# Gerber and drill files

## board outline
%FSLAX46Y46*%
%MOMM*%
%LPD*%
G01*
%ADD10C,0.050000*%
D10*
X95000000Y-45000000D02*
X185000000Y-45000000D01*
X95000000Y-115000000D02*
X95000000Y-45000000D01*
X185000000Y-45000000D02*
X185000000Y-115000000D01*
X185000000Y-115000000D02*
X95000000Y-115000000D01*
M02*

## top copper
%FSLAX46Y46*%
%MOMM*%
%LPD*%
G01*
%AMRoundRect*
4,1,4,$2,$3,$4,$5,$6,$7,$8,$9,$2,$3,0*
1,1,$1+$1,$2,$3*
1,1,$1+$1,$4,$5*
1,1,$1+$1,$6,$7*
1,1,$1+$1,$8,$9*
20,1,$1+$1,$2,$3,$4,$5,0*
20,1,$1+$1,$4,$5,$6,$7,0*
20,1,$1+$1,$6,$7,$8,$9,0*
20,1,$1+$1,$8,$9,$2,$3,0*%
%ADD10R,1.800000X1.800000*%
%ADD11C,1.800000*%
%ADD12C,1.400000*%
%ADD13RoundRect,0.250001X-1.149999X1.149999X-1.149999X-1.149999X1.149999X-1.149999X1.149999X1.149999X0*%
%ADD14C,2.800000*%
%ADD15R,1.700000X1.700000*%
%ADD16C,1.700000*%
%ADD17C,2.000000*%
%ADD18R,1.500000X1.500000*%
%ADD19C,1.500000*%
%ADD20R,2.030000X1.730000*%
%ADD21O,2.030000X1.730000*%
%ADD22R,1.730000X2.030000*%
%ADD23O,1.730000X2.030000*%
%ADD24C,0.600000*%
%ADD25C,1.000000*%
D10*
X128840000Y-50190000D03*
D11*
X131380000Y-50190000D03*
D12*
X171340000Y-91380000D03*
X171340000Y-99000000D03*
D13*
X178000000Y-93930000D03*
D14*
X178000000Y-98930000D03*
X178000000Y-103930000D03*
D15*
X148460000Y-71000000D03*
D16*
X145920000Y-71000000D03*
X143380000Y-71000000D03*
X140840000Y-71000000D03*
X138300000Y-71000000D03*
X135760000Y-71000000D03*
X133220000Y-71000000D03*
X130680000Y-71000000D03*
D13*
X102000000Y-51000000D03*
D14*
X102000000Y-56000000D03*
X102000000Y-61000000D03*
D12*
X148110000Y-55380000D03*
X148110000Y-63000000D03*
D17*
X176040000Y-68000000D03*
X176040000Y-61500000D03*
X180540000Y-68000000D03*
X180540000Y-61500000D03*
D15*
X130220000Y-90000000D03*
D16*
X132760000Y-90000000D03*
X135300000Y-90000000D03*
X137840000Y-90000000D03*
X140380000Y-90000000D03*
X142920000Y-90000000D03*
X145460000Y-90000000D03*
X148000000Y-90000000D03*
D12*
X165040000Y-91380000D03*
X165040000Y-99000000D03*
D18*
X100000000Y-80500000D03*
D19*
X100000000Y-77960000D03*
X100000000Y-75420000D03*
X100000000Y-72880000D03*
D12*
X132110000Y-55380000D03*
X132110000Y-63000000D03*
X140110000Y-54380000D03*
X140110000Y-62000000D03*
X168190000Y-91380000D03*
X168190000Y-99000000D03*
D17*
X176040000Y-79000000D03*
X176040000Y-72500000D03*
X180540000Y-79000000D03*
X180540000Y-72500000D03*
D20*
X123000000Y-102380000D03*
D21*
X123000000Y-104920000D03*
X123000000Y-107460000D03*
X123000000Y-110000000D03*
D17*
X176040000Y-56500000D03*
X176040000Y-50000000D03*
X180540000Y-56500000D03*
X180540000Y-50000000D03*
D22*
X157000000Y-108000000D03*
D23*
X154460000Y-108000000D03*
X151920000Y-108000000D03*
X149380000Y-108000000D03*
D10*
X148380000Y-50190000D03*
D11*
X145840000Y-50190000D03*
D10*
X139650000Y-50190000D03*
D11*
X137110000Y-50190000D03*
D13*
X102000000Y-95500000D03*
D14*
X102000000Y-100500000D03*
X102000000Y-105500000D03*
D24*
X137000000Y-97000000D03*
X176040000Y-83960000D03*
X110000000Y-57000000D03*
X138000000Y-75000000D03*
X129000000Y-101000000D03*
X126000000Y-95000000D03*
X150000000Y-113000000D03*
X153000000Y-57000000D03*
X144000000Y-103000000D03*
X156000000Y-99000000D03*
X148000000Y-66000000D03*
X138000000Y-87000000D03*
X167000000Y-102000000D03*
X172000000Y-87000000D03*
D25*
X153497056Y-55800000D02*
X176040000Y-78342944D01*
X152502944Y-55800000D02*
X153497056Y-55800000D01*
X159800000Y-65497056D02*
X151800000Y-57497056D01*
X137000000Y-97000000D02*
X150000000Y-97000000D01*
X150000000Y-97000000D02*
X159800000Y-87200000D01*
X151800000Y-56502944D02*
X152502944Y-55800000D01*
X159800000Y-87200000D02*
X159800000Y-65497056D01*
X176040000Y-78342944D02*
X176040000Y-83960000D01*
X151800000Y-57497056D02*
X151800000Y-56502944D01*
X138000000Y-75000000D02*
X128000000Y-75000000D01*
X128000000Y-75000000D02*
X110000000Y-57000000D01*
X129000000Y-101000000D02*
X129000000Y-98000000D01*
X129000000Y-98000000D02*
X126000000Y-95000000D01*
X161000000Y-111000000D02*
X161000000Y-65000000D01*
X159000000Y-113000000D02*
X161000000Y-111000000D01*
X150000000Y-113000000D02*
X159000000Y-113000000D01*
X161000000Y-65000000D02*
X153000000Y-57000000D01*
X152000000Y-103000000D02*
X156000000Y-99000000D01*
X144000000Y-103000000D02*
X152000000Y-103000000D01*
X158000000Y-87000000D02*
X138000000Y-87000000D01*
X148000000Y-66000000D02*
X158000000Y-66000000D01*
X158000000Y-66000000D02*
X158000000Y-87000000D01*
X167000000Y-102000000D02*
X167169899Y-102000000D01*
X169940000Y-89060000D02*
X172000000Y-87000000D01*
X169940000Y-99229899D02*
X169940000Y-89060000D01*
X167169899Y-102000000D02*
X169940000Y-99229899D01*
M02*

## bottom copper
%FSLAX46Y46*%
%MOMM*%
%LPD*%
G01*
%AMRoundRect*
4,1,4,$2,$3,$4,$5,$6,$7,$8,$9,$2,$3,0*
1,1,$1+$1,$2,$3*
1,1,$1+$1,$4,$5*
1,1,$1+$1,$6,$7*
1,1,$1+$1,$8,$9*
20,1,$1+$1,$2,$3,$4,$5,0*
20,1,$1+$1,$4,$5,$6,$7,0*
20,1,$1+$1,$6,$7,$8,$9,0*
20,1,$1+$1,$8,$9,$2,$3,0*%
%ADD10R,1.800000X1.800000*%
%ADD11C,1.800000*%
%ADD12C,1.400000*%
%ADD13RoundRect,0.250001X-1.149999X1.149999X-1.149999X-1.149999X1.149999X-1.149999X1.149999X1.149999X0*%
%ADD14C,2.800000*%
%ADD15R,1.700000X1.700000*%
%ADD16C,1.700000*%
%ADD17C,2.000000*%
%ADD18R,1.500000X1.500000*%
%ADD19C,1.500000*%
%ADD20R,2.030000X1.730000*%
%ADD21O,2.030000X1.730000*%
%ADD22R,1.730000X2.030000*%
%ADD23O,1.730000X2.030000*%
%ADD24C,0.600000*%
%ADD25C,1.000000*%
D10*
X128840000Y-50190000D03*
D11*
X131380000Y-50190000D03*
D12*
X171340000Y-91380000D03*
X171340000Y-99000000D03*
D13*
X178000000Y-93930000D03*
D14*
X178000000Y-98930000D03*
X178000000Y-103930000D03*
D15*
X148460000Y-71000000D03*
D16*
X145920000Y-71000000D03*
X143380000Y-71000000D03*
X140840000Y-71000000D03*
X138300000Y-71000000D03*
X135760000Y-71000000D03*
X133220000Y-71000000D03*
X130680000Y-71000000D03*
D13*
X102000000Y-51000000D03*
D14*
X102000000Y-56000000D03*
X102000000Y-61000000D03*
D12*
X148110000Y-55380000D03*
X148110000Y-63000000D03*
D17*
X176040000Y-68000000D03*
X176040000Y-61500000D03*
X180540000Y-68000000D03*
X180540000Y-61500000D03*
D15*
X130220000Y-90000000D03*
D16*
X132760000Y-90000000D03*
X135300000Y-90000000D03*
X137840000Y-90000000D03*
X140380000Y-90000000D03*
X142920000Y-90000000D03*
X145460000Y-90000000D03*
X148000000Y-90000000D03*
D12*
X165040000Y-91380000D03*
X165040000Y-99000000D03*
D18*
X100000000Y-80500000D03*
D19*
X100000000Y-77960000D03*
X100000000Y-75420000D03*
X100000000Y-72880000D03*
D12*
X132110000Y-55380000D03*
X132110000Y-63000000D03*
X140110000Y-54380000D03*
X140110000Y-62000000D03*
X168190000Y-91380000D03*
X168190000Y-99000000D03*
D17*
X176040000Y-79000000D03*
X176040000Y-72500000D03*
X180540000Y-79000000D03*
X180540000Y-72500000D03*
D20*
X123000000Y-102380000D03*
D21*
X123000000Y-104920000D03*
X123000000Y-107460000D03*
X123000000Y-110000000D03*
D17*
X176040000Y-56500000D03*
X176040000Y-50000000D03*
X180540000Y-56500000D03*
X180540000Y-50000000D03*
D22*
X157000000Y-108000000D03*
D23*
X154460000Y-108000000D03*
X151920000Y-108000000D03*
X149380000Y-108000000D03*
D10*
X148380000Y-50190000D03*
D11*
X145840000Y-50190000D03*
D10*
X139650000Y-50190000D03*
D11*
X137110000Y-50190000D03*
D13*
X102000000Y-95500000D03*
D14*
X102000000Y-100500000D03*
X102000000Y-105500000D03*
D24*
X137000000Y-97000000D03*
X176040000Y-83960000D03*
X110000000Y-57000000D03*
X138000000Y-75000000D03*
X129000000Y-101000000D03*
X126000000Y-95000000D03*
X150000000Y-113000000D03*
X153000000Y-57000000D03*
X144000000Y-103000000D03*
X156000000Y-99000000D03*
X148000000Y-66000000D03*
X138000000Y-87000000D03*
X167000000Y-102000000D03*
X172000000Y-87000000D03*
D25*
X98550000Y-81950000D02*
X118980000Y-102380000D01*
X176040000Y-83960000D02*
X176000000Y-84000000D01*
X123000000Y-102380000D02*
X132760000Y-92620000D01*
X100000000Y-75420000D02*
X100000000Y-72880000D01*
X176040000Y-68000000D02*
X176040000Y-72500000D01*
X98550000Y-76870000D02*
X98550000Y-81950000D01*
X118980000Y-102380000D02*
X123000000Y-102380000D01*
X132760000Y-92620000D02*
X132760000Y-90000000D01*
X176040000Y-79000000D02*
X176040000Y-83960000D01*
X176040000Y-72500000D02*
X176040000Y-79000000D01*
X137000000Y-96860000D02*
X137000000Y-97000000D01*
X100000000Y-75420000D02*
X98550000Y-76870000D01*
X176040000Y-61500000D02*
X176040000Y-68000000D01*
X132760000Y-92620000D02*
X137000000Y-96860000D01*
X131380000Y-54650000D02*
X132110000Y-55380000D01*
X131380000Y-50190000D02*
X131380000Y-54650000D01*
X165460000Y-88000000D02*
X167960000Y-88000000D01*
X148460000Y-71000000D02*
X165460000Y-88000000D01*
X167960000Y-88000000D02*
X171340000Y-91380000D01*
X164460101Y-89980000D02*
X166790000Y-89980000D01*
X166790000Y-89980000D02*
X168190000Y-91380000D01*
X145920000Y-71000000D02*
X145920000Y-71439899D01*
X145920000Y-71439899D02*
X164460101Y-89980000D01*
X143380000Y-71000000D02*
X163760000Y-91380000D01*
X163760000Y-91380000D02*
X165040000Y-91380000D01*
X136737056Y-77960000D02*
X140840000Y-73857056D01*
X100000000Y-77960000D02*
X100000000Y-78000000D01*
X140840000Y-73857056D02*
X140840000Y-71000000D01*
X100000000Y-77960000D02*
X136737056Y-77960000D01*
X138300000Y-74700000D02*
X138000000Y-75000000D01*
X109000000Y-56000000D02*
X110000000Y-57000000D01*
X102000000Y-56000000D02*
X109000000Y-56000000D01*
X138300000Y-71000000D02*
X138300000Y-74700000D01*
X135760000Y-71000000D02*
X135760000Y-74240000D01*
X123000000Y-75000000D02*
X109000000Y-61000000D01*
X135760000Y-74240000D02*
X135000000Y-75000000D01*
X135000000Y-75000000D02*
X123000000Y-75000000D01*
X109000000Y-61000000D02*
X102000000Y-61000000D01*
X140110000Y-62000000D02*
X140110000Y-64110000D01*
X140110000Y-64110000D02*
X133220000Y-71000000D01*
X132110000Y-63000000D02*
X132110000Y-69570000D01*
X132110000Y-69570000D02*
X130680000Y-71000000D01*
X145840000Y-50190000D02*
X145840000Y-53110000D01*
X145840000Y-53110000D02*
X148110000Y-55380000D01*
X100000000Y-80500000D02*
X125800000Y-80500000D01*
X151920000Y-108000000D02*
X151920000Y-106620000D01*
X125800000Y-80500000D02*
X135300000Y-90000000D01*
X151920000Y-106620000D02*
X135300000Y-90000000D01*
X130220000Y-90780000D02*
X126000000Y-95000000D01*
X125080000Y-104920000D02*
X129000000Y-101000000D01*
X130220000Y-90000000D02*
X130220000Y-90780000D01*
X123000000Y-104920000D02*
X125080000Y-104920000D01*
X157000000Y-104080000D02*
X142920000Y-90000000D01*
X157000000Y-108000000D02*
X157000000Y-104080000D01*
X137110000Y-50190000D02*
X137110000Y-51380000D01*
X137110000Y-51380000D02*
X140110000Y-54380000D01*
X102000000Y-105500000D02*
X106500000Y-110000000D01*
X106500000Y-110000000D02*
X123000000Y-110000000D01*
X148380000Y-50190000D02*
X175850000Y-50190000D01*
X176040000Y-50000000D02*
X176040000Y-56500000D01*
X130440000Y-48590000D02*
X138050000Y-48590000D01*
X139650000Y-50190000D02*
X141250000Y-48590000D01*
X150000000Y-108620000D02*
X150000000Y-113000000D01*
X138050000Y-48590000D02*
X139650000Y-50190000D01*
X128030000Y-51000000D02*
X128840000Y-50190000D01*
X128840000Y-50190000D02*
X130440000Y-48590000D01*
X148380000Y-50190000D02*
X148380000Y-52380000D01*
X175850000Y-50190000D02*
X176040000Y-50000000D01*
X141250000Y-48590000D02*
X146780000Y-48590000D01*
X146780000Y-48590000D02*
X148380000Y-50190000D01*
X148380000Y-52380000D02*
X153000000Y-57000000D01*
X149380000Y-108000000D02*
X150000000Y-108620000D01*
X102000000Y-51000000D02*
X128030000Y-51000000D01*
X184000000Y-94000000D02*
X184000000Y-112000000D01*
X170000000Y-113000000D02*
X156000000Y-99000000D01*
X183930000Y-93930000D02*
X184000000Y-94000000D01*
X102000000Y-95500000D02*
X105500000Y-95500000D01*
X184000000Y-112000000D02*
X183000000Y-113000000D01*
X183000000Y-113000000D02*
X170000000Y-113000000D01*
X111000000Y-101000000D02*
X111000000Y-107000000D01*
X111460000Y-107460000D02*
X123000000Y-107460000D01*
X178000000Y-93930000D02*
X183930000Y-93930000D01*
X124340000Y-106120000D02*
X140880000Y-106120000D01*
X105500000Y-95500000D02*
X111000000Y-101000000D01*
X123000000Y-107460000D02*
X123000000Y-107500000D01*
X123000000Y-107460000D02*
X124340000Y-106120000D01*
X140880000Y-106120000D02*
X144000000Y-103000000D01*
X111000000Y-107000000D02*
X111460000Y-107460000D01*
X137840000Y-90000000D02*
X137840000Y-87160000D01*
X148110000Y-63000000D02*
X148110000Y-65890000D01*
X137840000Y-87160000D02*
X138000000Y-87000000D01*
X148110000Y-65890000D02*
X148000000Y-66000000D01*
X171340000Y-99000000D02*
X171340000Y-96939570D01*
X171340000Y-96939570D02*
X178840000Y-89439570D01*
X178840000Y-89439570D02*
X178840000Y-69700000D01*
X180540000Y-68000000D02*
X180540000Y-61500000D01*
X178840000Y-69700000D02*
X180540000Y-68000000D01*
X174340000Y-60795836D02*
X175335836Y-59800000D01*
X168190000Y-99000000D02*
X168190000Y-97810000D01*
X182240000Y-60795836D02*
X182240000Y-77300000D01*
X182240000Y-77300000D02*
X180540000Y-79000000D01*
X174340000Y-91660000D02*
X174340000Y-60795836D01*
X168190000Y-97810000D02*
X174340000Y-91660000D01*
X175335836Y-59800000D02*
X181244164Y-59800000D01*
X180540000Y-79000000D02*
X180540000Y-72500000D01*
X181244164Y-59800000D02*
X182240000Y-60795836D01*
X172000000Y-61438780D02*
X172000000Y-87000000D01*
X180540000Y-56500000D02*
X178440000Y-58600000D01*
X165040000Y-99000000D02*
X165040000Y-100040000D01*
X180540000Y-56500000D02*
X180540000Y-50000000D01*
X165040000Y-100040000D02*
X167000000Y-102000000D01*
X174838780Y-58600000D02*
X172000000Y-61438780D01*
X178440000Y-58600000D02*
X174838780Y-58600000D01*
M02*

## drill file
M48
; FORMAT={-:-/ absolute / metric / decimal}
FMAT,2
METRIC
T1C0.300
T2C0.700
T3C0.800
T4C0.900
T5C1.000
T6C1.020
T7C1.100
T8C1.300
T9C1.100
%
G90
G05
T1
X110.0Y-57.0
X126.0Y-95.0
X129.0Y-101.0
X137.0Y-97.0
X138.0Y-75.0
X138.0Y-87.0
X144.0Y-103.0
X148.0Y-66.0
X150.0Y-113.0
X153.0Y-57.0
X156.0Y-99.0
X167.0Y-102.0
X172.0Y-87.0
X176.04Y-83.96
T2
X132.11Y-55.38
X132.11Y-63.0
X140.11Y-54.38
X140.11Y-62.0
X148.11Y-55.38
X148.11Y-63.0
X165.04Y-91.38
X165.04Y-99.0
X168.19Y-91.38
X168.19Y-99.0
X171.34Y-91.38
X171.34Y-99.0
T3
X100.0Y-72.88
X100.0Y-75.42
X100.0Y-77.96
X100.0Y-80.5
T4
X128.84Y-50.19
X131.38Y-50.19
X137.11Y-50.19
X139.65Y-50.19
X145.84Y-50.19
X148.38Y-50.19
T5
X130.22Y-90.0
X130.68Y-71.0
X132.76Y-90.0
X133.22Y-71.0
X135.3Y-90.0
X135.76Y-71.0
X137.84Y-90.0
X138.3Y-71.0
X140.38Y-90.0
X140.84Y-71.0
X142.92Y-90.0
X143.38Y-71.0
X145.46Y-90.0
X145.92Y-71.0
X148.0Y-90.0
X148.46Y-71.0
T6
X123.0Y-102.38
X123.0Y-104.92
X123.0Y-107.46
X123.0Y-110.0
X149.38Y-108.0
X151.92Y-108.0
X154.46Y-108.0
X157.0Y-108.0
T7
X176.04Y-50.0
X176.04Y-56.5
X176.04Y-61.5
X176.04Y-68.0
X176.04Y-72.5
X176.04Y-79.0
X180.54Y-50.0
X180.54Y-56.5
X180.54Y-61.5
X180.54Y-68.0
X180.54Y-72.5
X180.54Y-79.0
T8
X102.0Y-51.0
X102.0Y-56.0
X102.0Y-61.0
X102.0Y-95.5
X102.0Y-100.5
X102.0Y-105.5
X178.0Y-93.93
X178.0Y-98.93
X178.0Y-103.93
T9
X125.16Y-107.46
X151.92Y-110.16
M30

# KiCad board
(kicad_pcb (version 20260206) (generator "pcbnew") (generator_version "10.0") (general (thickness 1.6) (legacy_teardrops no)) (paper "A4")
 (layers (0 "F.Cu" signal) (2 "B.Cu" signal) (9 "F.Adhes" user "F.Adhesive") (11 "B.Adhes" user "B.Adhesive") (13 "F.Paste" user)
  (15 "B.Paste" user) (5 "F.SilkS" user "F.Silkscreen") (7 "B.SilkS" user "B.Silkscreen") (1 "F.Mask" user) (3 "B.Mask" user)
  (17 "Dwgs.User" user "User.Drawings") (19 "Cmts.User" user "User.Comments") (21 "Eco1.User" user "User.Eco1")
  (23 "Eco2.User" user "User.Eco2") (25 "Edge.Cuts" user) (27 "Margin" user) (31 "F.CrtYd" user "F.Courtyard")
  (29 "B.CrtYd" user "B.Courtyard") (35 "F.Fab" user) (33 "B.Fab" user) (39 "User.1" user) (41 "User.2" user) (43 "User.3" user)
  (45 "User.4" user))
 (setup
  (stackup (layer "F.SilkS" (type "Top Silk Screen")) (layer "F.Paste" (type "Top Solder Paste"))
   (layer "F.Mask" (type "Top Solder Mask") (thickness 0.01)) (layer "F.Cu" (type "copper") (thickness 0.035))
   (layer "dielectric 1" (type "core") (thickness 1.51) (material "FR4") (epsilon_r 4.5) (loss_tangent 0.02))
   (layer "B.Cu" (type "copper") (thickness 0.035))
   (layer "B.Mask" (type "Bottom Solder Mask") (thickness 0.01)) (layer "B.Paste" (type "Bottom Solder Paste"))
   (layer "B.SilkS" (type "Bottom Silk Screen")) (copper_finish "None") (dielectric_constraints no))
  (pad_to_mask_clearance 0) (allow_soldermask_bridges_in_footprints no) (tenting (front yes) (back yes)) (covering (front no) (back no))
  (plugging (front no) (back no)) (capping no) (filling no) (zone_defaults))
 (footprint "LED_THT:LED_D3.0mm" (layer "F.Cu") (at 128.84 50.19)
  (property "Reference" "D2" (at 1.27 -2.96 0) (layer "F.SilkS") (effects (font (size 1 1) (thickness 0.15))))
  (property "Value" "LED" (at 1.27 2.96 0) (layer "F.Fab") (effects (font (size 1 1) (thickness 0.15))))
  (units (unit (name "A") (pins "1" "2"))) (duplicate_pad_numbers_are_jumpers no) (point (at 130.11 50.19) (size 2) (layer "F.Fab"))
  (pad "1" thru_hole rect (at 0 0) (size 1.8 1.8) (drill 0.9) (layers "*.Cu" "*.Mask") (remove_unused_layers no) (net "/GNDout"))
  (pad "2" thru_hole circle (at 2.54 0) (size 1.8 1.8) (drill 0.9) (layers "*.Cu" "*.Mask") (remove_unused_layers no) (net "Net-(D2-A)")))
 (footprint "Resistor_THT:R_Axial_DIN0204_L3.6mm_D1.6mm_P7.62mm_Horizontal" (layer "F.Cu") (at 171.34 91.38 -90)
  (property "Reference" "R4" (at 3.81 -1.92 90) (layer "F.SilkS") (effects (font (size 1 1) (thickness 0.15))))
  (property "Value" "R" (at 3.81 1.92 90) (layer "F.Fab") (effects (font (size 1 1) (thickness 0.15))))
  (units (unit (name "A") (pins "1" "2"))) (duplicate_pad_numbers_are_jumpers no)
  (pad "1" thru_hole circle (at 0 0 270) (size 1.4 1.4) (drill 0.7) (layers "*.Cu" "*.Mask") (remove_unused_layers no) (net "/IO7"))
  (pad "2" thru_hole circle (at 7.62 0 270) (size 1.4 1.4) (drill 0.7) (layers "*.Cu" "*.Mask") (remove_unused_layers no)
   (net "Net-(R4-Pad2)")))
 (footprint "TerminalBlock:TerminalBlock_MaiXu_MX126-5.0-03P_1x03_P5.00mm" (layer "F.Cu") (at 178 93.93 -90)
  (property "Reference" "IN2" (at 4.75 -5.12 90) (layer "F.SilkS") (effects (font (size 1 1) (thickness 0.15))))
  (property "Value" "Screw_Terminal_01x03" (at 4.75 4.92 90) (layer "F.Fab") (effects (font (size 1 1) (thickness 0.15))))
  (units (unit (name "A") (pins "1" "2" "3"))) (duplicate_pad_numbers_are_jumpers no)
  (pad "1" thru_hole roundrect (at 0 0 270) (size 2.8 2.8) (drill 1.3) (layers "*.Cu" "*.Mask") (remove_unused_layers no)
   (roundrect_rratio 0.089286) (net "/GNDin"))
  (pad "2" thru_hole circle (at 5 0 270) (size 2.8 2.8) (drill 1.3) (layers "*.Cu" "*.Mask") (remove_unused_layers no)
   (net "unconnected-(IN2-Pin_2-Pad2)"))
  (pad "3" thru_hole circle (at 10 0 270) (size 2.8 2.8) (drill 1.3) (layers "*.Cu" "*.Mask") (remove_unused_layers no)
   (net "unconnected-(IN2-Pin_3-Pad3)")))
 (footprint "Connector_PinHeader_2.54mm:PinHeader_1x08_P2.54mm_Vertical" (layer "F.Cu") (at 148.46 71 -90)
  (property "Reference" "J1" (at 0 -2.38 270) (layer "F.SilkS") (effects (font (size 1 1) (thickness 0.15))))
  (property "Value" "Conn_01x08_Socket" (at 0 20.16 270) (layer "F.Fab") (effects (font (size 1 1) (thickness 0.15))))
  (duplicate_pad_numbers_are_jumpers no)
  (pad "1" thru_hole rect (at 0 0 270) (size 1.7 1.7) (drill 1) (layers "*.Cu" "*.Mask") (remove_unused_layers no) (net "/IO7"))
  (pad "2" thru_hole circle (at 0 2.54 270) (size 1.7 1.7) (drill 1) (layers "*.Cu" "*.Mask") (remove_unused_layers no) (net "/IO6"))
  (pad "3" thru_hole circle (at 0 5.08 270) (size 1.7 1.7) (drill 1) (layers "*.Cu" "*.Mask") (remove_unused_layers no) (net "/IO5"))
  (pad "4" thru_hole circle (at 0 7.62 270) (size 1.7 1.7) (drill 1) (layers "*.Cu" "*.Mask") (remove_unused_layers no) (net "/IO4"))
  (pad "5" thru_hole circle (at 0 10.16 270) (size 1.7 1.7) (drill 1) (layers "*.Cu" "*.Mask") (remove_unused_layers no) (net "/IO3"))
  (pad "6" thru_hole circle (at 0 12.7 270) (size 1.7 1.7) (drill 1) (layers "*.Cu" "*.Mask") (remove_unused_layers no) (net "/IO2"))
  (pad "7" thru_hole circle (at 0 15.24 270) (size 1.7 1.7) (drill 1) (layers "*.Cu" "*.Mask") (remove_unused_layers no) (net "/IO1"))
  (pad "8" thru_hole circle (at 0 17.78 270) (size 1.7 1.7) (drill 1) (layers "*.Cu" "*.Mask") (remove_unused_layers no) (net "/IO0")))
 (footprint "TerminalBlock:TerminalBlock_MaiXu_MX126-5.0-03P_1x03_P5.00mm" (layer "F.Cu") (at 102 51 -90)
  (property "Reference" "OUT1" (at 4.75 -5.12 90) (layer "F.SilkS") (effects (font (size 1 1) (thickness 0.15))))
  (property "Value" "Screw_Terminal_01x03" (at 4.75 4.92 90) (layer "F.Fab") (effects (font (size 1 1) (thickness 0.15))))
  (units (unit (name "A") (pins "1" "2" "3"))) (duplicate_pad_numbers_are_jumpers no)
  (pad "1" thru_hole roundrect (at 0 0 270) (size 2.8 2.8) (drill 1.3) (layers "*.Cu" "*.Mask") (remove_unused_layers no)
   (roundrect_rratio 0.089286) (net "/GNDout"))
  (pad "2" thru_hole circle (at 5 0 270) (size 2.8 2.8) (drill 1.3) (layers "*.Cu" "*.Mask") (remove_unused_layers no) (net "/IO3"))
  (pad "3" thru_hole circle (at 10 0 270) (size 2.8 2.8) (drill 1.3) (layers "*.Cu" "*.Mask") (remove_unused_layers no) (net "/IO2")))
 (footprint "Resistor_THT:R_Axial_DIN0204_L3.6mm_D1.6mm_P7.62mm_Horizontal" (layer "F.Cu") (at 148.11 55.38 -90)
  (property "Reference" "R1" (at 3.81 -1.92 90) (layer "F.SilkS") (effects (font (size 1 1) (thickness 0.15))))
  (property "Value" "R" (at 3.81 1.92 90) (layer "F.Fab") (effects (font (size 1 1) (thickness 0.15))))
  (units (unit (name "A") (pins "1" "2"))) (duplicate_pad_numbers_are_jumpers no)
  (pad "1" thru_hole circle (at 0 0 270) (size 1.4 1.4) (drill 0.7) (layers "*.Cu" "*.Mask") (remove_unused_layers no) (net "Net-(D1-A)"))
  (pad "2" thru_hole circle (at 7.62 0 270) (size 1.4 1.4) (drill 0.7) (layers "*.Cu" "*.Mask") (remove_unused_layers no) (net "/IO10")))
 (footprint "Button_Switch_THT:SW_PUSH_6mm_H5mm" (layer "F.Cu") (at 176.04 68 90)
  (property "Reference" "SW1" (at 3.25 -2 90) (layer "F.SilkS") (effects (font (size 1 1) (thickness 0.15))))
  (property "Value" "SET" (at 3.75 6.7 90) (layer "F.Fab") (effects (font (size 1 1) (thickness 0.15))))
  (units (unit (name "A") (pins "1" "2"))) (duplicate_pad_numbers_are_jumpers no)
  (pad "1" thru_hole circle (at 0 0 180) (size 2 2) (drill 1.1) (layers "*.Cu" "*.Mask") (remove_unused_layers no) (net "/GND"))
  (pad "1" thru_hole circle (at 6.5 0 180) (size 2 2) (drill 1.1) (layers "*.Cu" "*.Mask") (remove_unused_layers no) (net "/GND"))
  (pad "2" thru_hole circle (at 0 4.5 180) (size 2 2) (drill 1.1) (layers "*.Cu" "*.Mask") (remove_unused_layers no) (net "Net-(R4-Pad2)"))
  (pad "2" thru_hole circle (at 6.5 4.5 180) (size 2 2) (drill 1.1) (layers "*.Cu" "*.Mask") (remove_unused_layers no) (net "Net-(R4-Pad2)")))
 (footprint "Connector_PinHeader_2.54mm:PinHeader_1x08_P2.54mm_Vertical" (layer "F.Cu") (at 130.22 90 90)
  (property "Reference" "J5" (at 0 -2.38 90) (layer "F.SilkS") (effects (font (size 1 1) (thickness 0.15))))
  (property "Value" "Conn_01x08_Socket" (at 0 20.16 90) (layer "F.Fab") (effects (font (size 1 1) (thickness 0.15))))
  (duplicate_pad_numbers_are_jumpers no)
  (pad "1" thru_hole rect (at 0 0 90) (size 1.7 1.7) (drill 1) (layers "*.Cu" "*.Mask") (remove_unused_layers no) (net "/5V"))
  (pad "2" thru_hole circle (at 0 2.54 90) (size 1.7 1.7) (drill 1) (layers "*.Cu" "*.Mask") (remove_unused_layers no) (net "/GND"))
  (pad "3" thru_hole circle (at 0 5.08 90) (size 1.7 1.7) (drill 1) (layers "*.Cu" "*.Mask") (remove_unused_layers no) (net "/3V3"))
  (pad "4" thru_hole circle (at 0 7.62 90) (size 1.7 1.7) (drill 1) (layers "*.Cu" "*.Mask") (remove_unused_layers no) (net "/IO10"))
  (pad "5" thru_hole circle (at 0 10.16 90) (size 1.7 1.7) (drill 1) (layers "*.Cu" "*.Mask") (remove_unused_layers no) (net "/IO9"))
  (pad "6" thru_hole circle (at 0 12.7 90) (size 1.7 1.7) (drill 1) (layers "*.Cu" "*.Mask") (remove_unused_layers no) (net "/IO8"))
  (pad "7" thru_hole circle (at 0 15.24 90) (size 1.7 1.7) (drill 1) (layers "*.Cu" "*.Mask") (remove_unused_layers no) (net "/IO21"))
  (pad "8" thru_hole circle (at 0 17.78 90) (size 1.7 1.7) (drill 1) (layers "*.Cu" "*.Mask") (remove_unused_layers no) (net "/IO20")))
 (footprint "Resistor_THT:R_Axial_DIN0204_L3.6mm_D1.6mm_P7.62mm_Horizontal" (layer "F.Cu") (at 165.04 91.38 -90)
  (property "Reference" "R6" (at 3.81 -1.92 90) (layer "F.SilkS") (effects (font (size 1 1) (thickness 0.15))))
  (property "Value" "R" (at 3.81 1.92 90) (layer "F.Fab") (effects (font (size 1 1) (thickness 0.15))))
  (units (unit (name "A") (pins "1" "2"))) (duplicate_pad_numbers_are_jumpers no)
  (pad "1" thru_hole circle (at 0 0 270) (size 1.4 1.4) (drill 0.7) (layers "*.Cu" "*.Mask") (remove_unused_layers no) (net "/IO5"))
  (pad "2" thru_hole circle (at 7.62 0 270) (size 1.4 1.4) (drill 0.7) (layers "*.Cu" "*.Mask") (remove_unused_layers no)
   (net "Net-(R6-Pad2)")))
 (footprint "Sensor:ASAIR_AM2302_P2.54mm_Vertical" (layer "F.Cu") (at 100 80.5 90)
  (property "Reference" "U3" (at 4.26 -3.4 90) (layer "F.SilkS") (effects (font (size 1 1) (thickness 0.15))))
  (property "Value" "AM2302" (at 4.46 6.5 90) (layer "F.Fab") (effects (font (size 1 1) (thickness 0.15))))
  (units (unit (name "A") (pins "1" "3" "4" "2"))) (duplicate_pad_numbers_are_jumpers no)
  (pad "1" thru_hole rect (at 0 0 180) (size 1.5 1.5) (drill 0.8) (layers "*.Cu" "*.Mask") (remove_unused_layers no) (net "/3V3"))
  (pad "2" thru_hole circle (at 2.54 0 180) (size 1.5 1.5) (drill 0.8) (layers "*.Cu" "*.Mask") (remove_unused_layers no) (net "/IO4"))
  (pad "3" thru_hole circle (at 5.08 0 180) (size 1.5 1.5) (drill 0.8) (layers "*.Cu" "*.Mask") (remove_unused_layers no) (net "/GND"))
  (pad "4" thru_hole circle (at 7.62 0 180) (size 1.5 1.5) (drill 0.8) (layers "*.Cu" "*.Mask") (remove_unused_layers no) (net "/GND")))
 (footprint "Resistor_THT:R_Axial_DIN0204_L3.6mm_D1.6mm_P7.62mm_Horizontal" (layer "F.Cu") (at 132.11 55.38 -90)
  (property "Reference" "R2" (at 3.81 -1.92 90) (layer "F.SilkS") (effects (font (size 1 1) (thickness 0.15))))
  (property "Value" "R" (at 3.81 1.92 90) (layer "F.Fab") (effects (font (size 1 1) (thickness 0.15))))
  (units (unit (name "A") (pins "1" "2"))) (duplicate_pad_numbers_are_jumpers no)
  (pad "1" thru_hole circle (at 0 0 270) (size 1.4 1.4) (drill 0.7) (layers "*.Cu" "*.Mask") (remove_unused_layers no) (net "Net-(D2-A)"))
  (pad "2" thru_hole circle (at 7.62 0 270) (size 1.4 1.4) (drill 0.7) (layers "*.Cu" "*.Mask") (remove_unused_layers no) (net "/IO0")))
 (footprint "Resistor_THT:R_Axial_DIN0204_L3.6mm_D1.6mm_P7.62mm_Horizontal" (layer "F.Cu") (at 140.11 54.38 -90)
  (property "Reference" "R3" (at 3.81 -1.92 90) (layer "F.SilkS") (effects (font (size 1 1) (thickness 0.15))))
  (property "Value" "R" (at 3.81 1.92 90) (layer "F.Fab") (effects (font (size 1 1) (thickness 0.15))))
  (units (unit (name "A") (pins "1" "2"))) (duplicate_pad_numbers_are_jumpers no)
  (pad "1" thru_hole circle (at 0 0 270) (size 1.4 1.4) (drill 0.7) (layers "*.Cu" "*.Mask") (remove_unused_layers no) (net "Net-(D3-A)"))
  (pad "2" thru_hole circle (at 7.62 0 270) (size 1.4 1.4) (drill 0.7) (layers "*.Cu" "*.Mask") (remove_unused_layers no) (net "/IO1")))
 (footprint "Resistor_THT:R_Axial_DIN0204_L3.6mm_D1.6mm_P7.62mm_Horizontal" (layer "F.Cu") (at 168.19 91.38 -90)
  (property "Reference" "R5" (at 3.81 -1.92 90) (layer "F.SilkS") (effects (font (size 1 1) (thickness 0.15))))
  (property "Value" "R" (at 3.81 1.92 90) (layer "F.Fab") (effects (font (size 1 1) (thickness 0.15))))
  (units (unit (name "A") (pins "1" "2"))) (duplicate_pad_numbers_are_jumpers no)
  (pad "1" thru_hole circle (at 0 0 270) (size 1.4 1.4) (drill 0.7) (layers "*.Cu" "*.Mask") (remove_unused_layers no) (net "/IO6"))
  (pad "2" thru_hole circle (at 7.62 0 270) (size 1.4 1.4) (drill 0.7) (layers "*.Cu" "*.Mask") (remove_unused_layers no)
   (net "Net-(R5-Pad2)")))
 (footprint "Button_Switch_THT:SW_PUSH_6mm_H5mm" (layer "F.Cu") (at 176.04 79 90)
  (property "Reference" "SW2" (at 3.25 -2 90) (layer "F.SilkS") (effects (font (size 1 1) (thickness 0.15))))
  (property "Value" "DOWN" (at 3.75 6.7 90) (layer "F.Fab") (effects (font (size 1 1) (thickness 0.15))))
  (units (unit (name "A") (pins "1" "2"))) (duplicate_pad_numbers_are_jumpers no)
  (pad "1" thru_hole circle (at 0 0 180) (size 2 2) (drill 1.1) (layers "*.Cu" "*.Mask") (remove_unused_layers no) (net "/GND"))
  (pad "1" thru_hole circle (at 6.5 0 180) (size 2 2) (drill 1.1) (layers "*.Cu" "*.Mask") (remove_unused_layers no) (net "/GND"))
  (pad "2" thru_hole circle (at 0 4.5 180) (size 2 2) (drill 1.1) (layers "*.Cu" "*.Mask") (remove_unused_layers no) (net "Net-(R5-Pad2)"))
  (pad "2" thru_hole circle (at 6.5 4.5 180) (size 2 2) (drill 1.1) (layers "*.Cu" "*.Mask") (remove_unused_layers no) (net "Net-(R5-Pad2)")))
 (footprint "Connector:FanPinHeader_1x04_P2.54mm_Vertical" (layer "F.Cu") (at 123 102.38 -90)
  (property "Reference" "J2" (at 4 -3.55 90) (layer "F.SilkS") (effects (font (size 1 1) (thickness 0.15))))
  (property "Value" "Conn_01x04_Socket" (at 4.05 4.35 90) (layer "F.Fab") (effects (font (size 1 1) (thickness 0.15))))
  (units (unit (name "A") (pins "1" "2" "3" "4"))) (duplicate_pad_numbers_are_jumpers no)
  (pad "" np_thru_hole circle (at 5.08 -2.16) (size 1.1 1.1) (drill 1.1) (layers "*.Cu" "*.Mask"))
  (pad "1" thru_hole rect (at 0 0) (size 2.03 1.73) (drill 1.02) (layers "*.Cu" "*.Mask") (remove_unused_layers no) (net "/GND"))
  (pad "2" thru_hole oval (at 2.54 0) (size 2.03 1.73) (drill 1.02) (layers "*.Cu" "*.Mask") (remove_unused_layers no) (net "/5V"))
  (pad "3" thru_hole oval (at 5.08 0) (size 2.03 1.73) (drill 1.02) (layers "*.Cu" "*.Mask") (remove_unused_layers no) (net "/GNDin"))
  (pad "4" thru_hole oval (at 7.62 0) (size 2.03 1.73) (drill 1.02) (layers "*.Cu" "*.Mask") (remove_unused_layers no) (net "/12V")))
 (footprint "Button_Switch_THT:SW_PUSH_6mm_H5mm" (layer "F.Cu") (at 176.04 56.5 90)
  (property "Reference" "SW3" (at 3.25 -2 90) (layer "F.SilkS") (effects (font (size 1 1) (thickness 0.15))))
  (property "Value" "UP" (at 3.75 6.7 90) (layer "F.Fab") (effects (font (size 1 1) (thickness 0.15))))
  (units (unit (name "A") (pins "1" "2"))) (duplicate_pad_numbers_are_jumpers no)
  (pad "1" thru_hole circle (at 0 0 180) (size 2 2) (drill 1.1) (layers "*.Cu" "*.Mask") (remove_unused_layers no) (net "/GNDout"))
  (pad "1" thru_hole circle (at 6.5 0 180) (size 2 2) (drill 1.1) (layers "*.Cu" "*.Mask") (remove_unused_layers no) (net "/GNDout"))
  (pad "2" thru_hole circle (at 0 4.5 180) (size 2 2) (drill 1.1) (layers "*.Cu" "*.Mask") (remove_unused_layers no) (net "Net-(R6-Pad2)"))
  (pad "2" thru_hole circle (at 6.5 4.5 180) (size 2 2) (drill 1.1) (layers "*.Cu" "*.Mask") (remove_unused_layers no) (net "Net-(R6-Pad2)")))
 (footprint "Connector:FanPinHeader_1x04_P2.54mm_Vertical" (layer "F.Cu") (at 157 108 180)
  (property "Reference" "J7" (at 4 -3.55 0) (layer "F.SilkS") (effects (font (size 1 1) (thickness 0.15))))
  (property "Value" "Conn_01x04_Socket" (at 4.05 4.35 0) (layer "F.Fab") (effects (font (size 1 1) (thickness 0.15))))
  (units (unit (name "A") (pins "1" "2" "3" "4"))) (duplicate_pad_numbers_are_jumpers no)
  (pad "" np_thru_hole circle (at 5.08 -2.16 270) (size 1.1 1.1) (drill 1.1) (layers "*.Cu" "*.Mask"))
  (pad "1" thru_hole rect (at 0 0 270) (size 2.03 1.73) (drill 1.02) (layers "*.Cu" "*.Mask") (remove_unused_layers no) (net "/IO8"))
  (pad "2" thru_hole oval (at 2.54 0 270) (size 2.03 1.73) (drill 1.02) (layers "*.Cu" "*.Mask") (remove_unused_layers no)
   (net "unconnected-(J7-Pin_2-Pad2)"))
  (pad "3" thru_hole oval (at 5.08 0 270) (size 2.03 1.73) (drill 1.02) (layers "*.Cu" "*.Mask") (remove_unused_layers no) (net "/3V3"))
  (pad "4" thru_hole oval (at 7.62 0 270) (size 2.03 1.73) (drill 1.02) (layers "*.Cu" "*.Mask") (remove_unused_layers no) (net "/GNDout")))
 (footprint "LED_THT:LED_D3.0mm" (layer "F.Cu") (at 148.38 50.19 180)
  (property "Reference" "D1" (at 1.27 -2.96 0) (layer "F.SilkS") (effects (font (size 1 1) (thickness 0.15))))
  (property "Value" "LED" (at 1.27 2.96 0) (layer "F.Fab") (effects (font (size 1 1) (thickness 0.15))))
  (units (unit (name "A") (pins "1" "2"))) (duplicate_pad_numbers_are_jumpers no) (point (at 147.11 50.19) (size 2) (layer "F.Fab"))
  (pad "1" thru_hole rect (at 0 0 180) (size 1.8 1.8) (drill 0.9) (layers "*.Cu" "*.Mask") (remove_unused_layers no) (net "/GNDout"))
  (pad "2" thru_hole circle (at 2.54 0 180) (size 1.8 1.8) (drill 0.9) (layers "*.Cu" "*.Mask") (remove_unused_layers no) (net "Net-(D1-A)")))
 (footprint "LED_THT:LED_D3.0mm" (layer "F.Cu") (at 139.65 50.19 180)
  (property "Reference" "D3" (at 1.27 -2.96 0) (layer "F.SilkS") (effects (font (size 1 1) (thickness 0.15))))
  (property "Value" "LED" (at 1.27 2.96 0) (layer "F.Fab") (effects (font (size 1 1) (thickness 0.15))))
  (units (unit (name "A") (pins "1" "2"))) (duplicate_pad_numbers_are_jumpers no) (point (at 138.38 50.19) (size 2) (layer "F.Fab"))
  (pad "1" thru_hole rect (at 0 0 180) (size 1.8 1.8) (drill 0.9) (layers "*.Cu" "*.Mask") (remove_unused_layers no) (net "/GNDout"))
  (pad "2" thru_hole circle (at 2.54 0 180) (size 1.8 1.8) (drill 0.9) (layers "*.Cu" "*.Mask") (remove_unused_layers no) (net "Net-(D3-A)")))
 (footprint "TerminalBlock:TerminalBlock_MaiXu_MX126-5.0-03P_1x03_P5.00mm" (layer "F.Cu") (at 102 95.5 -90)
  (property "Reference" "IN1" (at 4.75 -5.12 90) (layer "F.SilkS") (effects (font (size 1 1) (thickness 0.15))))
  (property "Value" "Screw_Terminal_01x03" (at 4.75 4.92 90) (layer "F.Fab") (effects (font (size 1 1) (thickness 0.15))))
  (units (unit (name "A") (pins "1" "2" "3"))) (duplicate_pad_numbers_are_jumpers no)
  (pad "1" thru_hole roundrect (at 0 0 270) (size 2.8 2.8) (drill 1.3) (layers "*.Cu" "*.Mask") (remove_unused_layers no)
   (roundrect_rratio 0.089286) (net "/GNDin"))
  (pad "2" thru_hole circle (at 5 0 270) (size 2.8 2.8) (drill 1.3) (layers "*.Cu" "*.Mask") (remove_unused_layers no)
   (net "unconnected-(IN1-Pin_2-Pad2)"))
  (pad "3" thru_hole circle (at 10 0 270) (size 2.8 2.8) (drill 1.3) (layers "*.Cu" "*.Mask") (remove_unused_layers no) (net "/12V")))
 (gr_line (start 95 45) (end 185 45) (stroke (width 0.05) (type default)) (layer "Edge.Cuts"))
 (gr_line (start 95 115) (end 95 45) (stroke (width 0.05) (type default)) (layer "Edge.Cuts"))
 (gr_line (start 185 45) (end 185 115) (stroke (width 0.05) (type default)) (layer "Edge.Cuts"))
 (gr_line (start 185 115) (end 95 115) (stroke (width 0.05) (type default)) (layer "Edge.Cuts"))
 (segment (start 153.497056 55.8) (end 176.04 78.342944) (width 1) (layer "F.Cu") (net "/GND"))
 (segment (start 152.502944 55.8) (end 153.497056 55.8) (width 1) (layer "F.Cu") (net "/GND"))
 (segment (start 159.8 65.497056) (end 151.8 57.497056) (width 1) (layer "F.Cu") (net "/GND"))
 (segment (start 137 97) (end 150 97) (width 1) (layer "F.Cu") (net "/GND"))
 (segment (start 150 97) (end 159.8 87.2) (width 1) (layer "F.Cu") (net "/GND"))
 (segment (start 151.8 56.502944) (end 152.502944 55.8) (width 1) (layer "F.Cu") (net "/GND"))
 (segment (start 159.8 87.2) (end 159.8 65.497056) (width 1) (layer "F.Cu") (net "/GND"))
 (segment (start 176.04 78.342944) (end 176.04 83.96) (width 1) (layer "F.Cu") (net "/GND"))
 (segment (start 151.8 57.497056) (end 151.8 56.502944) (width 1) (layer "F.Cu") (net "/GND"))
 (via (at 137 97) (size 0.6) (drill 0.3) (layers "F.Cu" "B.Cu") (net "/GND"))
 (via (at 176.04 83.96) (size 0.6) (drill 0.3) (layers "F.Cu" "B.Cu") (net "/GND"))
 (segment (start 98.55 81.95) (end 118.98 102.38) (width 1) (layer "B.Cu") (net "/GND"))
 (segment (start 176.04 83.96) (end 176 84) (width 1) (layer "B.Cu") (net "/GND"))
 (segment (start 123 102.38) (end 132.76 92.62) (width 1) (layer "B.Cu") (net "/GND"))
 (segment (start 100 75.42) (end 100 72.88) (width 1) (layer "B.Cu") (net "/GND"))
 (segment (start 176.04 68) (end 176.04 72.5) (width 1) (layer "B.Cu") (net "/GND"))
 (segment (start 98.55 76.87) (end 98.55 81.95) (width 1) (layer "B.Cu") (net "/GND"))
 (segment (start 118.98 102.38) (end 123 102.38) (width 1) (layer "B.Cu") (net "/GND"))
 (segment (start 132.76 92.62) (end 132.76 90) (width 1) (layer "B.Cu") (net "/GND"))
 (segment (start 176.04 79) (end 176.04 83.96) (width 1) (layer "B.Cu") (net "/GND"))
 (segment (start 176.04 72.5) (end 176.04 79) (width 1) (layer "B.Cu") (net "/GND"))
 (segment (start 137 96.86) (end 137 97) (width 1) (layer "B.Cu") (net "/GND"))
 (segment (start 100 75.42) (end 98.55 76.87) (width 1) (layer "B.Cu") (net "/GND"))
 (segment (start 176.04 61.5) (end 176.04 68) (width 1) (layer "B.Cu") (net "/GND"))
 (segment (start 132.76 92.62) (end 137 96.86) (width 1) (layer "B.Cu") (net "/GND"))
 (segment (start 131.38 54.65) (end 132.11 55.38) (width 1) (layer "B.Cu") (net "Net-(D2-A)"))
 (segment (start 131.38 50.19) (end 131.38 54.65) (width 1) (layer "B.Cu") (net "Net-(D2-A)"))
 (segment (start 165.46 88) (end 167.96 88) (width 1) (layer "B.Cu") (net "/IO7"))
 (segment (start 148.46 71) (end 165.46 88) (width 1) (layer "B.Cu") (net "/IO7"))
 (segment (start 167.96 88) (end 171.34 91.38) (width 1) (layer "B.Cu") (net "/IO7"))
 (segment (start 164.460101 89.98) (end 166.79 89.98) (width 1) (layer "B.Cu") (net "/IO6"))
 (segment (start 166.79 89.98) (end 168.19 91.38) (width 1) (layer "B.Cu") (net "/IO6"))
 (segment (start 145.92 71) (end 145.92 71.439899) (width 1) (layer "B.Cu") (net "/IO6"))
 (segment (start 145.92 71.439899) (end 164.460101 89.98) (width 1) (layer "B.Cu") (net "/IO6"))
 (segment (start 143.38 71) (end 163.76 91.38) (width 1) (layer "B.Cu") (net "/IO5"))
 (segment (start 163.76 91.38) (end 165.04 91.38) (width 1) (layer "B.Cu") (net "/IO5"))
 (segment (start 136.737056 77.96) (end 140.84 73.857056) (width 1) (layer "B.Cu") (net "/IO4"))
 (segment (start 100 77.96) (end 100 78) (width 1) (layer "B.Cu") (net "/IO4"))
 (segment (start 140.84 73.857056) (end 140.84 71) (width 1) (layer "B.Cu") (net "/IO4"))
 (segment (start 100 77.96) (end 136.737056 77.96) (width 1) (layer "B.Cu") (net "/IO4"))
 (segment (start 138 75) (end 128 75) (width 1) (layer "F.Cu") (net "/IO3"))
 (segment (start 128 75) (end 110 57) (width 1) (layer "F.Cu") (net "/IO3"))
 (via (at 110 57) (size 0.6) (drill 0.3) (layers "F.Cu" "B.Cu") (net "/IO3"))
 (via (at 138 75) (size 0.6) (drill 0.3) (layers "F.Cu" "B.Cu") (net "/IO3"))
 (segment (start 138.3 74.7) (end 138 75) (width 1) (layer "B.Cu") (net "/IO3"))
 (segment (start 109 56) (end 110 57) (width 1) (layer "B.Cu") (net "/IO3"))
 (segment (start 102 56) (end 109 56) (width 1) (layer "B.Cu") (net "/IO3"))
 (segment (start 138.3 71) (end 138.3 74.7) (width 1) (layer "B.Cu") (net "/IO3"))
 (segment (start 135.76 71) (end 135.76 74.24) (width 1) (layer "B.Cu") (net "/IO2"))
 (segment (start 123 75) (end 109 61) (width 1) (layer "B.Cu") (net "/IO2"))
 (segment (start 135.76 74.24) (end 135 75) (width 1) (layer "B.Cu") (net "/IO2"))
 (segment (start 135 75) (end 123 75) (width 1) (layer "B.Cu") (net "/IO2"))
 (segment (start 109 61) (end 102 61) (width 1) (layer "B.Cu") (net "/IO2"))
 (segment (start 140.11 62) (end 140.11 64.11) (width 1) (layer "B.Cu") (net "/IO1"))
 (segment (start 140.11 64.11) (end 133.22 71) (width 1) (layer "B.Cu") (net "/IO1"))
 (segment (start 132.11 63) (end 132.11 69.57) (width 1) (layer "B.Cu") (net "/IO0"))
 (segment (start 132.11 69.57) (end 130.68 71) (width 1) (layer "B.Cu") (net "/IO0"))
 (segment (start 145.84 50.19) (end 145.84 53.11) (width 1) (layer "B.Cu") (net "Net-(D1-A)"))
 (segment (start 145.84 53.11) (end 148.11 55.38) (width 1) (layer "B.Cu") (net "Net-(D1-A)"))
 (segment (start 100 80.5) (end 125.8 80.5) (width 1) (layer "B.Cu") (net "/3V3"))
 (segment (start 151.92 108) (end 151.92 106.62) (width 1) (layer "B.Cu") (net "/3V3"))
 (segment (start 125.8 80.5) (end 135.3 90) (width 1) (layer "B.Cu") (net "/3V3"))
 (segment (start 151.92 106.62) (end 135.3 90) (width 1) (layer "B.Cu") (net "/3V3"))
 (segment (start 129 101) (end 129 98) (width 1) (layer "F.Cu") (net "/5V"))
 (segment (start 129 98) (end 126 95) (width 1) (layer "F.Cu") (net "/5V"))
 (via (at 129 101) (size 0.6) (drill 0.3) (layers "F.Cu" "B.Cu") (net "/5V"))
 (via (at 126 95) (size 0.6) (drill 0.3) (layers "F.Cu" "B.Cu") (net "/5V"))
 (segment (start 130.22 90.78) (end 126 95) (width 1) (layer "B.Cu") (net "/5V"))
 (segment (start 125.08 104.92) (end 129 101) (width 1) (layer "B.Cu") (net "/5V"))
 (segment (start 130.22 90) (end 130.22 90.78) (width 1) (layer "B.Cu") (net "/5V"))
 (segment (start 123 104.92) (end 125.08 104.92) (width 1) (layer "B.Cu") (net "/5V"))
 (segment (start 157 104.08) (end 142.92 90) (width 1) (layer "B.Cu") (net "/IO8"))
 (segment (start 157 108) (end 157 104.08) (width 1) (layer "B.Cu") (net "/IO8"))
 (segment (start 137.11 50.19) (end 137.11 51.38) (width 1) (layer "B.Cu") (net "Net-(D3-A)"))
 (segment (start 137.11 51.38) (end 140.11 54.38) (width 1) (layer "B.Cu") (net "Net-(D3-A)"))
 (segment (start 102 105.5) (end 106.5 110) (width 1) (layer "B.Cu") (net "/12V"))
 (segment (start 106.5 110) (end 123 110) (width 1) (layer "B.Cu") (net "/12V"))
 (segment (start 161 111) (end 161 65) (width 1) (layer "F.Cu") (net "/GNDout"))
 (segment (start 159 113) (end 161 111) (width 1) (layer "F.Cu") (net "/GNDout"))
 (segment (start 150 113) (end 159 113) (width 1) (layer "F.Cu") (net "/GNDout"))
 (segment (start 161 65) (end 153 57) (width 1) (layer "F.Cu") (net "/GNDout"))
 (via (at 150 113) (size 0.6) (drill 0.3) (layers "F.Cu" "B.Cu") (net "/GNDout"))
 (via (at 153 57) (size 0.6) (drill 0.3) (layers "F.Cu" "B.Cu") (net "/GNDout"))
 (segment (start 148.38 50.19) (end 175.85 50.19) (width 1) (layer "B.Cu") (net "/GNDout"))
 (segment (start 176.04 50) (end 176.04 56.5) (width 1) (layer "B.Cu") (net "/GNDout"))
 (segment (start 130.44 48.59) (end 138.05 48.59) (width 1) (layer "B.Cu") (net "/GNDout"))
 (segment (start 139.65 50.19) (end 141.25 48.59) (width 1) (layer "B.Cu") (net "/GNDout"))
 (segment (start 150 108.62) (end 150 113) (width 1) (layer "B.Cu") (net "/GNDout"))
 (segment (start 138.05 48.59) (end 139.65 50.19) (width 1) (layer "B.Cu") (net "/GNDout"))
 (segment (start 128.03 51) (end 128.84 50.19) (width 1) (layer "B.Cu") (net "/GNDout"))
 (segment (start 128.84 50.19) (end 130.44 48.59) (width 1) (layer "B.Cu") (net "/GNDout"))
 (segment (start 148.38 50.19) (end 148.38 52.38) (width 1) (layer "B.Cu") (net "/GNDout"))
 (segment (start 175.85 50.19) (end 176.04 50) (width 1) (layer "B.Cu") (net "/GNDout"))
 (segment (start 141.25 48.59) (end 146.78 48.59) (width 1) (layer "B.Cu") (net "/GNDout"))
 (segment (start 146.78 48.59) (end 148.38 50.19) (width 1) (layer "B.Cu") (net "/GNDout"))
 (segment (start 148.38 52.38) (end 153 57) (width 1) (layer "B.Cu") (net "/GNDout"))
 (segment (start 149.38 108) (end 150 108.62) (width 1) (layer "B.Cu") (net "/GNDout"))
 (segment (start 102 51) (end 128.03 51) (width 1) (layer "B.Cu") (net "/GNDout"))
 (segment (start 152 103) (end 156 99) (width 1) (layer "F.Cu") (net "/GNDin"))
 (segment (start 144 103) (end 152 103) (width 1) (layer "F.Cu") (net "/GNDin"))
 (via (at 144 103) (size 0.6) (drill 0.3) (layers "F.Cu" "B.Cu") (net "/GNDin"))
 (via (at 156 99) (size 0.6) (drill 0.3) (layers "F.Cu" "B.Cu") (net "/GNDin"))
 (segment (start 184 94) (end 184 112) (width 1) (layer "B.Cu") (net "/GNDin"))
 (segment (start 170 113) (end 156 99) (width 1) (layer "B.Cu") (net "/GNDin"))
 (segment (start 183.93 93.93) (end 184 94) (width 1) (layer "B.Cu") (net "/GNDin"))
 (segment (start 102 95.5) (end 105.5 95.5) (width 1) (layer "B.Cu") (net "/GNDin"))
 (segment (start 184 112) (end 183 113) (width 1) (layer "B.Cu") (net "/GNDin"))
 (segment (start 183 113) (end 170 113) (width 1) (layer "B.Cu") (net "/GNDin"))
 (segment (start 111 101) (end 111 107) (width 1) (layer "B.Cu") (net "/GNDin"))
 (segment (start 111.46 107.46) (end 123 107.46) (width 1) (layer "B.Cu") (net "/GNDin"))
 (segment (start 178 93.93) (end 183.93 93.93) (width 1) (layer "B.Cu") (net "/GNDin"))
 (segment (start 124.34 106.12) (end 140.88 106.12) (width 1) (layer "B.Cu") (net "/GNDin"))
 (segment (start 105.5 95.5) (end 111 101) (width 1) (layer "B.Cu") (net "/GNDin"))
 (segment (start 123 107.46) (end 123 107.5) (width 1) (layer "B.Cu") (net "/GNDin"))
 (segment (start 123 107.46) (end 124.34 106.12) (width 1) (layer "B.Cu") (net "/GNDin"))
 (segment (start 140.88 106.12) (end 144 103) (width 1) (layer "B.Cu") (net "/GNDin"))
 (segment (start 111 107) (end 111.46 107.46) (width 1) (layer "B.Cu") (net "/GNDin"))
 (segment (start 158 87) (end 138 87) (width 1) (layer "F.Cu") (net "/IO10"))
 (segment (start 148 66) (end 158 66) (width 1) (layer "F.Cu") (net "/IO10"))
 (segment (start 158 66) (end 158 87) (width 1) (layer "F.Cu") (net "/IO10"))
 (via (at 148 66) (size 0.6) (drill 0.3) (layers "F.Cu" "B.Cu") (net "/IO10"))
 (via (at 138 87) (size 0.6) (drill 0.3) (layers "F.Cu" "B.Cu") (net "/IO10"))
 (segment (start 137.84 90) (end 137.84 87.16) (width 1) (layer "B.Cu") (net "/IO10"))
 (segment (start 148.11 63) (end 148.11 65.89) (width 1) (layer "B.Cu") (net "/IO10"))
 (segment (start 137.84 87.16) (end 138 87) (width 1) (layer "B.Cu") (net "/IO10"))
 (segment (start 148.11 65.89) (end 148 66) (width 1) (layer "B.Cu") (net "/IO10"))
 (segment (start 171.34 99) (end 171.34 96.93957) (width 1) (layer "B.Cu") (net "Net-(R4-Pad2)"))
 (segment (start 171.34 96.93957) (end 178.84 89.43957) (width 1) (layer "B.Cu") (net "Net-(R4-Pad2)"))
 (segment (start 178.84 89.43957) (end 178.84 69.7) (width 1) (layer "B.Cu") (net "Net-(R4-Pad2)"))
 (segment (start 180.54 68) (end 180.54 61.5) (width 1) (layer "B.Cu") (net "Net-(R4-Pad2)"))
 (segment (start 178.84 69.7) (end 180.54 68) (width 1) (layer "B.Cu") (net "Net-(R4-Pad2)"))
 (segment (start 174.34 60.795836) (end 175.335836 59.8) (width 1) (layer "B.Cu") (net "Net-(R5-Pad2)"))
 (segment (start 168.19 99) (end 168.19 97.81) (width 1) (layer "B.Cu") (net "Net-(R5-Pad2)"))
 (segment (start 182.24 60.795836) (end 182.24 77.3) (width 1) (layer "B.Cu") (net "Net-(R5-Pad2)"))
 (segment (start 182.24 77.3) (end 180.54 79) (width 1) (layer "B.Cu") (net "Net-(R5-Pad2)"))
 (segment (start 174.34 91.66) (end 174.34 60.795836) (width 1) (layer "B.Cu") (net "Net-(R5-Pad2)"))
 (segment (start 168.19 97.81) (end 174.34 91.66) (width 1) (layer "B.Cu") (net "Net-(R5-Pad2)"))
 (segment (start 175.335836 59.8) (end 181.244164 59.8) (width 1) (layer "B.Cu") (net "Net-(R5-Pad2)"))
 (segment (start 180.54 79) (end 180.54 72.5) (width 1) (layer "B.Cu") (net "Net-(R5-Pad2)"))
 (segment (start 181.244164 59.8) (end 182.24 60.795836) (width 1) (layer "B.Cu") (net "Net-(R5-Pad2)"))
 (segment (start 167 102) (end 167.169899 102) (width 1) (layer "F.Cu") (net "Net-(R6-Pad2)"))
 (segment (start 169.94 89.06) (end 172 87) (width 1) (layer "F.Cu") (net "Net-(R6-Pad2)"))
 (segment (start 169.94 99.229899) (end 169.94 89.06) (width 1) (layer "F.Cu") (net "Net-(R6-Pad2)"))
 (segment (start 167.169899 102) (end 169.94 99.229899) (width 1) (layer "F.Cu") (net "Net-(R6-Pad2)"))
 (via (at 167 102) (size 0.6) (drill 0.3) (layers "F.Cu" "B.Cu") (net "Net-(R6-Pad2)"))
 (via (at 172 87) (size 0.6) (drill 0.3) (layers "F.Cu" "B.Cu") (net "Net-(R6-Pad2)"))
 (segment (start 172 61.43878) (end 172 87) (width 1) (layer "B.Cu") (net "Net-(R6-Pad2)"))
 (segment (start 180.54 56.5) (end 178.44 58.6) (width 1) (layer "B.Cu") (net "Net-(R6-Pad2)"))
 (segment (start 165.04 99) (end 165.04 100.04) (width 1) (layer "B.Cu") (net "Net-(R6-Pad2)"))
 (segment (start 180.54 56.5) (end 180.54 50) (width 1) (layer "B.Cu") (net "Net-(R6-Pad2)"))
 (segment (start 165.04 100.04) (end 167 102) (width 1) (layer "B.Cu") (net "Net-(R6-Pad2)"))
 (segment (start 174.83878 58.6) (end 172 61.43878) (width 1) (layer "B.Cu") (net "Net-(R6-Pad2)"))
 (segment (start 178.44 58.6) (end 174.83878 58.6) (width 1) (layer "B.Cu") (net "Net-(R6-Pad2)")))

